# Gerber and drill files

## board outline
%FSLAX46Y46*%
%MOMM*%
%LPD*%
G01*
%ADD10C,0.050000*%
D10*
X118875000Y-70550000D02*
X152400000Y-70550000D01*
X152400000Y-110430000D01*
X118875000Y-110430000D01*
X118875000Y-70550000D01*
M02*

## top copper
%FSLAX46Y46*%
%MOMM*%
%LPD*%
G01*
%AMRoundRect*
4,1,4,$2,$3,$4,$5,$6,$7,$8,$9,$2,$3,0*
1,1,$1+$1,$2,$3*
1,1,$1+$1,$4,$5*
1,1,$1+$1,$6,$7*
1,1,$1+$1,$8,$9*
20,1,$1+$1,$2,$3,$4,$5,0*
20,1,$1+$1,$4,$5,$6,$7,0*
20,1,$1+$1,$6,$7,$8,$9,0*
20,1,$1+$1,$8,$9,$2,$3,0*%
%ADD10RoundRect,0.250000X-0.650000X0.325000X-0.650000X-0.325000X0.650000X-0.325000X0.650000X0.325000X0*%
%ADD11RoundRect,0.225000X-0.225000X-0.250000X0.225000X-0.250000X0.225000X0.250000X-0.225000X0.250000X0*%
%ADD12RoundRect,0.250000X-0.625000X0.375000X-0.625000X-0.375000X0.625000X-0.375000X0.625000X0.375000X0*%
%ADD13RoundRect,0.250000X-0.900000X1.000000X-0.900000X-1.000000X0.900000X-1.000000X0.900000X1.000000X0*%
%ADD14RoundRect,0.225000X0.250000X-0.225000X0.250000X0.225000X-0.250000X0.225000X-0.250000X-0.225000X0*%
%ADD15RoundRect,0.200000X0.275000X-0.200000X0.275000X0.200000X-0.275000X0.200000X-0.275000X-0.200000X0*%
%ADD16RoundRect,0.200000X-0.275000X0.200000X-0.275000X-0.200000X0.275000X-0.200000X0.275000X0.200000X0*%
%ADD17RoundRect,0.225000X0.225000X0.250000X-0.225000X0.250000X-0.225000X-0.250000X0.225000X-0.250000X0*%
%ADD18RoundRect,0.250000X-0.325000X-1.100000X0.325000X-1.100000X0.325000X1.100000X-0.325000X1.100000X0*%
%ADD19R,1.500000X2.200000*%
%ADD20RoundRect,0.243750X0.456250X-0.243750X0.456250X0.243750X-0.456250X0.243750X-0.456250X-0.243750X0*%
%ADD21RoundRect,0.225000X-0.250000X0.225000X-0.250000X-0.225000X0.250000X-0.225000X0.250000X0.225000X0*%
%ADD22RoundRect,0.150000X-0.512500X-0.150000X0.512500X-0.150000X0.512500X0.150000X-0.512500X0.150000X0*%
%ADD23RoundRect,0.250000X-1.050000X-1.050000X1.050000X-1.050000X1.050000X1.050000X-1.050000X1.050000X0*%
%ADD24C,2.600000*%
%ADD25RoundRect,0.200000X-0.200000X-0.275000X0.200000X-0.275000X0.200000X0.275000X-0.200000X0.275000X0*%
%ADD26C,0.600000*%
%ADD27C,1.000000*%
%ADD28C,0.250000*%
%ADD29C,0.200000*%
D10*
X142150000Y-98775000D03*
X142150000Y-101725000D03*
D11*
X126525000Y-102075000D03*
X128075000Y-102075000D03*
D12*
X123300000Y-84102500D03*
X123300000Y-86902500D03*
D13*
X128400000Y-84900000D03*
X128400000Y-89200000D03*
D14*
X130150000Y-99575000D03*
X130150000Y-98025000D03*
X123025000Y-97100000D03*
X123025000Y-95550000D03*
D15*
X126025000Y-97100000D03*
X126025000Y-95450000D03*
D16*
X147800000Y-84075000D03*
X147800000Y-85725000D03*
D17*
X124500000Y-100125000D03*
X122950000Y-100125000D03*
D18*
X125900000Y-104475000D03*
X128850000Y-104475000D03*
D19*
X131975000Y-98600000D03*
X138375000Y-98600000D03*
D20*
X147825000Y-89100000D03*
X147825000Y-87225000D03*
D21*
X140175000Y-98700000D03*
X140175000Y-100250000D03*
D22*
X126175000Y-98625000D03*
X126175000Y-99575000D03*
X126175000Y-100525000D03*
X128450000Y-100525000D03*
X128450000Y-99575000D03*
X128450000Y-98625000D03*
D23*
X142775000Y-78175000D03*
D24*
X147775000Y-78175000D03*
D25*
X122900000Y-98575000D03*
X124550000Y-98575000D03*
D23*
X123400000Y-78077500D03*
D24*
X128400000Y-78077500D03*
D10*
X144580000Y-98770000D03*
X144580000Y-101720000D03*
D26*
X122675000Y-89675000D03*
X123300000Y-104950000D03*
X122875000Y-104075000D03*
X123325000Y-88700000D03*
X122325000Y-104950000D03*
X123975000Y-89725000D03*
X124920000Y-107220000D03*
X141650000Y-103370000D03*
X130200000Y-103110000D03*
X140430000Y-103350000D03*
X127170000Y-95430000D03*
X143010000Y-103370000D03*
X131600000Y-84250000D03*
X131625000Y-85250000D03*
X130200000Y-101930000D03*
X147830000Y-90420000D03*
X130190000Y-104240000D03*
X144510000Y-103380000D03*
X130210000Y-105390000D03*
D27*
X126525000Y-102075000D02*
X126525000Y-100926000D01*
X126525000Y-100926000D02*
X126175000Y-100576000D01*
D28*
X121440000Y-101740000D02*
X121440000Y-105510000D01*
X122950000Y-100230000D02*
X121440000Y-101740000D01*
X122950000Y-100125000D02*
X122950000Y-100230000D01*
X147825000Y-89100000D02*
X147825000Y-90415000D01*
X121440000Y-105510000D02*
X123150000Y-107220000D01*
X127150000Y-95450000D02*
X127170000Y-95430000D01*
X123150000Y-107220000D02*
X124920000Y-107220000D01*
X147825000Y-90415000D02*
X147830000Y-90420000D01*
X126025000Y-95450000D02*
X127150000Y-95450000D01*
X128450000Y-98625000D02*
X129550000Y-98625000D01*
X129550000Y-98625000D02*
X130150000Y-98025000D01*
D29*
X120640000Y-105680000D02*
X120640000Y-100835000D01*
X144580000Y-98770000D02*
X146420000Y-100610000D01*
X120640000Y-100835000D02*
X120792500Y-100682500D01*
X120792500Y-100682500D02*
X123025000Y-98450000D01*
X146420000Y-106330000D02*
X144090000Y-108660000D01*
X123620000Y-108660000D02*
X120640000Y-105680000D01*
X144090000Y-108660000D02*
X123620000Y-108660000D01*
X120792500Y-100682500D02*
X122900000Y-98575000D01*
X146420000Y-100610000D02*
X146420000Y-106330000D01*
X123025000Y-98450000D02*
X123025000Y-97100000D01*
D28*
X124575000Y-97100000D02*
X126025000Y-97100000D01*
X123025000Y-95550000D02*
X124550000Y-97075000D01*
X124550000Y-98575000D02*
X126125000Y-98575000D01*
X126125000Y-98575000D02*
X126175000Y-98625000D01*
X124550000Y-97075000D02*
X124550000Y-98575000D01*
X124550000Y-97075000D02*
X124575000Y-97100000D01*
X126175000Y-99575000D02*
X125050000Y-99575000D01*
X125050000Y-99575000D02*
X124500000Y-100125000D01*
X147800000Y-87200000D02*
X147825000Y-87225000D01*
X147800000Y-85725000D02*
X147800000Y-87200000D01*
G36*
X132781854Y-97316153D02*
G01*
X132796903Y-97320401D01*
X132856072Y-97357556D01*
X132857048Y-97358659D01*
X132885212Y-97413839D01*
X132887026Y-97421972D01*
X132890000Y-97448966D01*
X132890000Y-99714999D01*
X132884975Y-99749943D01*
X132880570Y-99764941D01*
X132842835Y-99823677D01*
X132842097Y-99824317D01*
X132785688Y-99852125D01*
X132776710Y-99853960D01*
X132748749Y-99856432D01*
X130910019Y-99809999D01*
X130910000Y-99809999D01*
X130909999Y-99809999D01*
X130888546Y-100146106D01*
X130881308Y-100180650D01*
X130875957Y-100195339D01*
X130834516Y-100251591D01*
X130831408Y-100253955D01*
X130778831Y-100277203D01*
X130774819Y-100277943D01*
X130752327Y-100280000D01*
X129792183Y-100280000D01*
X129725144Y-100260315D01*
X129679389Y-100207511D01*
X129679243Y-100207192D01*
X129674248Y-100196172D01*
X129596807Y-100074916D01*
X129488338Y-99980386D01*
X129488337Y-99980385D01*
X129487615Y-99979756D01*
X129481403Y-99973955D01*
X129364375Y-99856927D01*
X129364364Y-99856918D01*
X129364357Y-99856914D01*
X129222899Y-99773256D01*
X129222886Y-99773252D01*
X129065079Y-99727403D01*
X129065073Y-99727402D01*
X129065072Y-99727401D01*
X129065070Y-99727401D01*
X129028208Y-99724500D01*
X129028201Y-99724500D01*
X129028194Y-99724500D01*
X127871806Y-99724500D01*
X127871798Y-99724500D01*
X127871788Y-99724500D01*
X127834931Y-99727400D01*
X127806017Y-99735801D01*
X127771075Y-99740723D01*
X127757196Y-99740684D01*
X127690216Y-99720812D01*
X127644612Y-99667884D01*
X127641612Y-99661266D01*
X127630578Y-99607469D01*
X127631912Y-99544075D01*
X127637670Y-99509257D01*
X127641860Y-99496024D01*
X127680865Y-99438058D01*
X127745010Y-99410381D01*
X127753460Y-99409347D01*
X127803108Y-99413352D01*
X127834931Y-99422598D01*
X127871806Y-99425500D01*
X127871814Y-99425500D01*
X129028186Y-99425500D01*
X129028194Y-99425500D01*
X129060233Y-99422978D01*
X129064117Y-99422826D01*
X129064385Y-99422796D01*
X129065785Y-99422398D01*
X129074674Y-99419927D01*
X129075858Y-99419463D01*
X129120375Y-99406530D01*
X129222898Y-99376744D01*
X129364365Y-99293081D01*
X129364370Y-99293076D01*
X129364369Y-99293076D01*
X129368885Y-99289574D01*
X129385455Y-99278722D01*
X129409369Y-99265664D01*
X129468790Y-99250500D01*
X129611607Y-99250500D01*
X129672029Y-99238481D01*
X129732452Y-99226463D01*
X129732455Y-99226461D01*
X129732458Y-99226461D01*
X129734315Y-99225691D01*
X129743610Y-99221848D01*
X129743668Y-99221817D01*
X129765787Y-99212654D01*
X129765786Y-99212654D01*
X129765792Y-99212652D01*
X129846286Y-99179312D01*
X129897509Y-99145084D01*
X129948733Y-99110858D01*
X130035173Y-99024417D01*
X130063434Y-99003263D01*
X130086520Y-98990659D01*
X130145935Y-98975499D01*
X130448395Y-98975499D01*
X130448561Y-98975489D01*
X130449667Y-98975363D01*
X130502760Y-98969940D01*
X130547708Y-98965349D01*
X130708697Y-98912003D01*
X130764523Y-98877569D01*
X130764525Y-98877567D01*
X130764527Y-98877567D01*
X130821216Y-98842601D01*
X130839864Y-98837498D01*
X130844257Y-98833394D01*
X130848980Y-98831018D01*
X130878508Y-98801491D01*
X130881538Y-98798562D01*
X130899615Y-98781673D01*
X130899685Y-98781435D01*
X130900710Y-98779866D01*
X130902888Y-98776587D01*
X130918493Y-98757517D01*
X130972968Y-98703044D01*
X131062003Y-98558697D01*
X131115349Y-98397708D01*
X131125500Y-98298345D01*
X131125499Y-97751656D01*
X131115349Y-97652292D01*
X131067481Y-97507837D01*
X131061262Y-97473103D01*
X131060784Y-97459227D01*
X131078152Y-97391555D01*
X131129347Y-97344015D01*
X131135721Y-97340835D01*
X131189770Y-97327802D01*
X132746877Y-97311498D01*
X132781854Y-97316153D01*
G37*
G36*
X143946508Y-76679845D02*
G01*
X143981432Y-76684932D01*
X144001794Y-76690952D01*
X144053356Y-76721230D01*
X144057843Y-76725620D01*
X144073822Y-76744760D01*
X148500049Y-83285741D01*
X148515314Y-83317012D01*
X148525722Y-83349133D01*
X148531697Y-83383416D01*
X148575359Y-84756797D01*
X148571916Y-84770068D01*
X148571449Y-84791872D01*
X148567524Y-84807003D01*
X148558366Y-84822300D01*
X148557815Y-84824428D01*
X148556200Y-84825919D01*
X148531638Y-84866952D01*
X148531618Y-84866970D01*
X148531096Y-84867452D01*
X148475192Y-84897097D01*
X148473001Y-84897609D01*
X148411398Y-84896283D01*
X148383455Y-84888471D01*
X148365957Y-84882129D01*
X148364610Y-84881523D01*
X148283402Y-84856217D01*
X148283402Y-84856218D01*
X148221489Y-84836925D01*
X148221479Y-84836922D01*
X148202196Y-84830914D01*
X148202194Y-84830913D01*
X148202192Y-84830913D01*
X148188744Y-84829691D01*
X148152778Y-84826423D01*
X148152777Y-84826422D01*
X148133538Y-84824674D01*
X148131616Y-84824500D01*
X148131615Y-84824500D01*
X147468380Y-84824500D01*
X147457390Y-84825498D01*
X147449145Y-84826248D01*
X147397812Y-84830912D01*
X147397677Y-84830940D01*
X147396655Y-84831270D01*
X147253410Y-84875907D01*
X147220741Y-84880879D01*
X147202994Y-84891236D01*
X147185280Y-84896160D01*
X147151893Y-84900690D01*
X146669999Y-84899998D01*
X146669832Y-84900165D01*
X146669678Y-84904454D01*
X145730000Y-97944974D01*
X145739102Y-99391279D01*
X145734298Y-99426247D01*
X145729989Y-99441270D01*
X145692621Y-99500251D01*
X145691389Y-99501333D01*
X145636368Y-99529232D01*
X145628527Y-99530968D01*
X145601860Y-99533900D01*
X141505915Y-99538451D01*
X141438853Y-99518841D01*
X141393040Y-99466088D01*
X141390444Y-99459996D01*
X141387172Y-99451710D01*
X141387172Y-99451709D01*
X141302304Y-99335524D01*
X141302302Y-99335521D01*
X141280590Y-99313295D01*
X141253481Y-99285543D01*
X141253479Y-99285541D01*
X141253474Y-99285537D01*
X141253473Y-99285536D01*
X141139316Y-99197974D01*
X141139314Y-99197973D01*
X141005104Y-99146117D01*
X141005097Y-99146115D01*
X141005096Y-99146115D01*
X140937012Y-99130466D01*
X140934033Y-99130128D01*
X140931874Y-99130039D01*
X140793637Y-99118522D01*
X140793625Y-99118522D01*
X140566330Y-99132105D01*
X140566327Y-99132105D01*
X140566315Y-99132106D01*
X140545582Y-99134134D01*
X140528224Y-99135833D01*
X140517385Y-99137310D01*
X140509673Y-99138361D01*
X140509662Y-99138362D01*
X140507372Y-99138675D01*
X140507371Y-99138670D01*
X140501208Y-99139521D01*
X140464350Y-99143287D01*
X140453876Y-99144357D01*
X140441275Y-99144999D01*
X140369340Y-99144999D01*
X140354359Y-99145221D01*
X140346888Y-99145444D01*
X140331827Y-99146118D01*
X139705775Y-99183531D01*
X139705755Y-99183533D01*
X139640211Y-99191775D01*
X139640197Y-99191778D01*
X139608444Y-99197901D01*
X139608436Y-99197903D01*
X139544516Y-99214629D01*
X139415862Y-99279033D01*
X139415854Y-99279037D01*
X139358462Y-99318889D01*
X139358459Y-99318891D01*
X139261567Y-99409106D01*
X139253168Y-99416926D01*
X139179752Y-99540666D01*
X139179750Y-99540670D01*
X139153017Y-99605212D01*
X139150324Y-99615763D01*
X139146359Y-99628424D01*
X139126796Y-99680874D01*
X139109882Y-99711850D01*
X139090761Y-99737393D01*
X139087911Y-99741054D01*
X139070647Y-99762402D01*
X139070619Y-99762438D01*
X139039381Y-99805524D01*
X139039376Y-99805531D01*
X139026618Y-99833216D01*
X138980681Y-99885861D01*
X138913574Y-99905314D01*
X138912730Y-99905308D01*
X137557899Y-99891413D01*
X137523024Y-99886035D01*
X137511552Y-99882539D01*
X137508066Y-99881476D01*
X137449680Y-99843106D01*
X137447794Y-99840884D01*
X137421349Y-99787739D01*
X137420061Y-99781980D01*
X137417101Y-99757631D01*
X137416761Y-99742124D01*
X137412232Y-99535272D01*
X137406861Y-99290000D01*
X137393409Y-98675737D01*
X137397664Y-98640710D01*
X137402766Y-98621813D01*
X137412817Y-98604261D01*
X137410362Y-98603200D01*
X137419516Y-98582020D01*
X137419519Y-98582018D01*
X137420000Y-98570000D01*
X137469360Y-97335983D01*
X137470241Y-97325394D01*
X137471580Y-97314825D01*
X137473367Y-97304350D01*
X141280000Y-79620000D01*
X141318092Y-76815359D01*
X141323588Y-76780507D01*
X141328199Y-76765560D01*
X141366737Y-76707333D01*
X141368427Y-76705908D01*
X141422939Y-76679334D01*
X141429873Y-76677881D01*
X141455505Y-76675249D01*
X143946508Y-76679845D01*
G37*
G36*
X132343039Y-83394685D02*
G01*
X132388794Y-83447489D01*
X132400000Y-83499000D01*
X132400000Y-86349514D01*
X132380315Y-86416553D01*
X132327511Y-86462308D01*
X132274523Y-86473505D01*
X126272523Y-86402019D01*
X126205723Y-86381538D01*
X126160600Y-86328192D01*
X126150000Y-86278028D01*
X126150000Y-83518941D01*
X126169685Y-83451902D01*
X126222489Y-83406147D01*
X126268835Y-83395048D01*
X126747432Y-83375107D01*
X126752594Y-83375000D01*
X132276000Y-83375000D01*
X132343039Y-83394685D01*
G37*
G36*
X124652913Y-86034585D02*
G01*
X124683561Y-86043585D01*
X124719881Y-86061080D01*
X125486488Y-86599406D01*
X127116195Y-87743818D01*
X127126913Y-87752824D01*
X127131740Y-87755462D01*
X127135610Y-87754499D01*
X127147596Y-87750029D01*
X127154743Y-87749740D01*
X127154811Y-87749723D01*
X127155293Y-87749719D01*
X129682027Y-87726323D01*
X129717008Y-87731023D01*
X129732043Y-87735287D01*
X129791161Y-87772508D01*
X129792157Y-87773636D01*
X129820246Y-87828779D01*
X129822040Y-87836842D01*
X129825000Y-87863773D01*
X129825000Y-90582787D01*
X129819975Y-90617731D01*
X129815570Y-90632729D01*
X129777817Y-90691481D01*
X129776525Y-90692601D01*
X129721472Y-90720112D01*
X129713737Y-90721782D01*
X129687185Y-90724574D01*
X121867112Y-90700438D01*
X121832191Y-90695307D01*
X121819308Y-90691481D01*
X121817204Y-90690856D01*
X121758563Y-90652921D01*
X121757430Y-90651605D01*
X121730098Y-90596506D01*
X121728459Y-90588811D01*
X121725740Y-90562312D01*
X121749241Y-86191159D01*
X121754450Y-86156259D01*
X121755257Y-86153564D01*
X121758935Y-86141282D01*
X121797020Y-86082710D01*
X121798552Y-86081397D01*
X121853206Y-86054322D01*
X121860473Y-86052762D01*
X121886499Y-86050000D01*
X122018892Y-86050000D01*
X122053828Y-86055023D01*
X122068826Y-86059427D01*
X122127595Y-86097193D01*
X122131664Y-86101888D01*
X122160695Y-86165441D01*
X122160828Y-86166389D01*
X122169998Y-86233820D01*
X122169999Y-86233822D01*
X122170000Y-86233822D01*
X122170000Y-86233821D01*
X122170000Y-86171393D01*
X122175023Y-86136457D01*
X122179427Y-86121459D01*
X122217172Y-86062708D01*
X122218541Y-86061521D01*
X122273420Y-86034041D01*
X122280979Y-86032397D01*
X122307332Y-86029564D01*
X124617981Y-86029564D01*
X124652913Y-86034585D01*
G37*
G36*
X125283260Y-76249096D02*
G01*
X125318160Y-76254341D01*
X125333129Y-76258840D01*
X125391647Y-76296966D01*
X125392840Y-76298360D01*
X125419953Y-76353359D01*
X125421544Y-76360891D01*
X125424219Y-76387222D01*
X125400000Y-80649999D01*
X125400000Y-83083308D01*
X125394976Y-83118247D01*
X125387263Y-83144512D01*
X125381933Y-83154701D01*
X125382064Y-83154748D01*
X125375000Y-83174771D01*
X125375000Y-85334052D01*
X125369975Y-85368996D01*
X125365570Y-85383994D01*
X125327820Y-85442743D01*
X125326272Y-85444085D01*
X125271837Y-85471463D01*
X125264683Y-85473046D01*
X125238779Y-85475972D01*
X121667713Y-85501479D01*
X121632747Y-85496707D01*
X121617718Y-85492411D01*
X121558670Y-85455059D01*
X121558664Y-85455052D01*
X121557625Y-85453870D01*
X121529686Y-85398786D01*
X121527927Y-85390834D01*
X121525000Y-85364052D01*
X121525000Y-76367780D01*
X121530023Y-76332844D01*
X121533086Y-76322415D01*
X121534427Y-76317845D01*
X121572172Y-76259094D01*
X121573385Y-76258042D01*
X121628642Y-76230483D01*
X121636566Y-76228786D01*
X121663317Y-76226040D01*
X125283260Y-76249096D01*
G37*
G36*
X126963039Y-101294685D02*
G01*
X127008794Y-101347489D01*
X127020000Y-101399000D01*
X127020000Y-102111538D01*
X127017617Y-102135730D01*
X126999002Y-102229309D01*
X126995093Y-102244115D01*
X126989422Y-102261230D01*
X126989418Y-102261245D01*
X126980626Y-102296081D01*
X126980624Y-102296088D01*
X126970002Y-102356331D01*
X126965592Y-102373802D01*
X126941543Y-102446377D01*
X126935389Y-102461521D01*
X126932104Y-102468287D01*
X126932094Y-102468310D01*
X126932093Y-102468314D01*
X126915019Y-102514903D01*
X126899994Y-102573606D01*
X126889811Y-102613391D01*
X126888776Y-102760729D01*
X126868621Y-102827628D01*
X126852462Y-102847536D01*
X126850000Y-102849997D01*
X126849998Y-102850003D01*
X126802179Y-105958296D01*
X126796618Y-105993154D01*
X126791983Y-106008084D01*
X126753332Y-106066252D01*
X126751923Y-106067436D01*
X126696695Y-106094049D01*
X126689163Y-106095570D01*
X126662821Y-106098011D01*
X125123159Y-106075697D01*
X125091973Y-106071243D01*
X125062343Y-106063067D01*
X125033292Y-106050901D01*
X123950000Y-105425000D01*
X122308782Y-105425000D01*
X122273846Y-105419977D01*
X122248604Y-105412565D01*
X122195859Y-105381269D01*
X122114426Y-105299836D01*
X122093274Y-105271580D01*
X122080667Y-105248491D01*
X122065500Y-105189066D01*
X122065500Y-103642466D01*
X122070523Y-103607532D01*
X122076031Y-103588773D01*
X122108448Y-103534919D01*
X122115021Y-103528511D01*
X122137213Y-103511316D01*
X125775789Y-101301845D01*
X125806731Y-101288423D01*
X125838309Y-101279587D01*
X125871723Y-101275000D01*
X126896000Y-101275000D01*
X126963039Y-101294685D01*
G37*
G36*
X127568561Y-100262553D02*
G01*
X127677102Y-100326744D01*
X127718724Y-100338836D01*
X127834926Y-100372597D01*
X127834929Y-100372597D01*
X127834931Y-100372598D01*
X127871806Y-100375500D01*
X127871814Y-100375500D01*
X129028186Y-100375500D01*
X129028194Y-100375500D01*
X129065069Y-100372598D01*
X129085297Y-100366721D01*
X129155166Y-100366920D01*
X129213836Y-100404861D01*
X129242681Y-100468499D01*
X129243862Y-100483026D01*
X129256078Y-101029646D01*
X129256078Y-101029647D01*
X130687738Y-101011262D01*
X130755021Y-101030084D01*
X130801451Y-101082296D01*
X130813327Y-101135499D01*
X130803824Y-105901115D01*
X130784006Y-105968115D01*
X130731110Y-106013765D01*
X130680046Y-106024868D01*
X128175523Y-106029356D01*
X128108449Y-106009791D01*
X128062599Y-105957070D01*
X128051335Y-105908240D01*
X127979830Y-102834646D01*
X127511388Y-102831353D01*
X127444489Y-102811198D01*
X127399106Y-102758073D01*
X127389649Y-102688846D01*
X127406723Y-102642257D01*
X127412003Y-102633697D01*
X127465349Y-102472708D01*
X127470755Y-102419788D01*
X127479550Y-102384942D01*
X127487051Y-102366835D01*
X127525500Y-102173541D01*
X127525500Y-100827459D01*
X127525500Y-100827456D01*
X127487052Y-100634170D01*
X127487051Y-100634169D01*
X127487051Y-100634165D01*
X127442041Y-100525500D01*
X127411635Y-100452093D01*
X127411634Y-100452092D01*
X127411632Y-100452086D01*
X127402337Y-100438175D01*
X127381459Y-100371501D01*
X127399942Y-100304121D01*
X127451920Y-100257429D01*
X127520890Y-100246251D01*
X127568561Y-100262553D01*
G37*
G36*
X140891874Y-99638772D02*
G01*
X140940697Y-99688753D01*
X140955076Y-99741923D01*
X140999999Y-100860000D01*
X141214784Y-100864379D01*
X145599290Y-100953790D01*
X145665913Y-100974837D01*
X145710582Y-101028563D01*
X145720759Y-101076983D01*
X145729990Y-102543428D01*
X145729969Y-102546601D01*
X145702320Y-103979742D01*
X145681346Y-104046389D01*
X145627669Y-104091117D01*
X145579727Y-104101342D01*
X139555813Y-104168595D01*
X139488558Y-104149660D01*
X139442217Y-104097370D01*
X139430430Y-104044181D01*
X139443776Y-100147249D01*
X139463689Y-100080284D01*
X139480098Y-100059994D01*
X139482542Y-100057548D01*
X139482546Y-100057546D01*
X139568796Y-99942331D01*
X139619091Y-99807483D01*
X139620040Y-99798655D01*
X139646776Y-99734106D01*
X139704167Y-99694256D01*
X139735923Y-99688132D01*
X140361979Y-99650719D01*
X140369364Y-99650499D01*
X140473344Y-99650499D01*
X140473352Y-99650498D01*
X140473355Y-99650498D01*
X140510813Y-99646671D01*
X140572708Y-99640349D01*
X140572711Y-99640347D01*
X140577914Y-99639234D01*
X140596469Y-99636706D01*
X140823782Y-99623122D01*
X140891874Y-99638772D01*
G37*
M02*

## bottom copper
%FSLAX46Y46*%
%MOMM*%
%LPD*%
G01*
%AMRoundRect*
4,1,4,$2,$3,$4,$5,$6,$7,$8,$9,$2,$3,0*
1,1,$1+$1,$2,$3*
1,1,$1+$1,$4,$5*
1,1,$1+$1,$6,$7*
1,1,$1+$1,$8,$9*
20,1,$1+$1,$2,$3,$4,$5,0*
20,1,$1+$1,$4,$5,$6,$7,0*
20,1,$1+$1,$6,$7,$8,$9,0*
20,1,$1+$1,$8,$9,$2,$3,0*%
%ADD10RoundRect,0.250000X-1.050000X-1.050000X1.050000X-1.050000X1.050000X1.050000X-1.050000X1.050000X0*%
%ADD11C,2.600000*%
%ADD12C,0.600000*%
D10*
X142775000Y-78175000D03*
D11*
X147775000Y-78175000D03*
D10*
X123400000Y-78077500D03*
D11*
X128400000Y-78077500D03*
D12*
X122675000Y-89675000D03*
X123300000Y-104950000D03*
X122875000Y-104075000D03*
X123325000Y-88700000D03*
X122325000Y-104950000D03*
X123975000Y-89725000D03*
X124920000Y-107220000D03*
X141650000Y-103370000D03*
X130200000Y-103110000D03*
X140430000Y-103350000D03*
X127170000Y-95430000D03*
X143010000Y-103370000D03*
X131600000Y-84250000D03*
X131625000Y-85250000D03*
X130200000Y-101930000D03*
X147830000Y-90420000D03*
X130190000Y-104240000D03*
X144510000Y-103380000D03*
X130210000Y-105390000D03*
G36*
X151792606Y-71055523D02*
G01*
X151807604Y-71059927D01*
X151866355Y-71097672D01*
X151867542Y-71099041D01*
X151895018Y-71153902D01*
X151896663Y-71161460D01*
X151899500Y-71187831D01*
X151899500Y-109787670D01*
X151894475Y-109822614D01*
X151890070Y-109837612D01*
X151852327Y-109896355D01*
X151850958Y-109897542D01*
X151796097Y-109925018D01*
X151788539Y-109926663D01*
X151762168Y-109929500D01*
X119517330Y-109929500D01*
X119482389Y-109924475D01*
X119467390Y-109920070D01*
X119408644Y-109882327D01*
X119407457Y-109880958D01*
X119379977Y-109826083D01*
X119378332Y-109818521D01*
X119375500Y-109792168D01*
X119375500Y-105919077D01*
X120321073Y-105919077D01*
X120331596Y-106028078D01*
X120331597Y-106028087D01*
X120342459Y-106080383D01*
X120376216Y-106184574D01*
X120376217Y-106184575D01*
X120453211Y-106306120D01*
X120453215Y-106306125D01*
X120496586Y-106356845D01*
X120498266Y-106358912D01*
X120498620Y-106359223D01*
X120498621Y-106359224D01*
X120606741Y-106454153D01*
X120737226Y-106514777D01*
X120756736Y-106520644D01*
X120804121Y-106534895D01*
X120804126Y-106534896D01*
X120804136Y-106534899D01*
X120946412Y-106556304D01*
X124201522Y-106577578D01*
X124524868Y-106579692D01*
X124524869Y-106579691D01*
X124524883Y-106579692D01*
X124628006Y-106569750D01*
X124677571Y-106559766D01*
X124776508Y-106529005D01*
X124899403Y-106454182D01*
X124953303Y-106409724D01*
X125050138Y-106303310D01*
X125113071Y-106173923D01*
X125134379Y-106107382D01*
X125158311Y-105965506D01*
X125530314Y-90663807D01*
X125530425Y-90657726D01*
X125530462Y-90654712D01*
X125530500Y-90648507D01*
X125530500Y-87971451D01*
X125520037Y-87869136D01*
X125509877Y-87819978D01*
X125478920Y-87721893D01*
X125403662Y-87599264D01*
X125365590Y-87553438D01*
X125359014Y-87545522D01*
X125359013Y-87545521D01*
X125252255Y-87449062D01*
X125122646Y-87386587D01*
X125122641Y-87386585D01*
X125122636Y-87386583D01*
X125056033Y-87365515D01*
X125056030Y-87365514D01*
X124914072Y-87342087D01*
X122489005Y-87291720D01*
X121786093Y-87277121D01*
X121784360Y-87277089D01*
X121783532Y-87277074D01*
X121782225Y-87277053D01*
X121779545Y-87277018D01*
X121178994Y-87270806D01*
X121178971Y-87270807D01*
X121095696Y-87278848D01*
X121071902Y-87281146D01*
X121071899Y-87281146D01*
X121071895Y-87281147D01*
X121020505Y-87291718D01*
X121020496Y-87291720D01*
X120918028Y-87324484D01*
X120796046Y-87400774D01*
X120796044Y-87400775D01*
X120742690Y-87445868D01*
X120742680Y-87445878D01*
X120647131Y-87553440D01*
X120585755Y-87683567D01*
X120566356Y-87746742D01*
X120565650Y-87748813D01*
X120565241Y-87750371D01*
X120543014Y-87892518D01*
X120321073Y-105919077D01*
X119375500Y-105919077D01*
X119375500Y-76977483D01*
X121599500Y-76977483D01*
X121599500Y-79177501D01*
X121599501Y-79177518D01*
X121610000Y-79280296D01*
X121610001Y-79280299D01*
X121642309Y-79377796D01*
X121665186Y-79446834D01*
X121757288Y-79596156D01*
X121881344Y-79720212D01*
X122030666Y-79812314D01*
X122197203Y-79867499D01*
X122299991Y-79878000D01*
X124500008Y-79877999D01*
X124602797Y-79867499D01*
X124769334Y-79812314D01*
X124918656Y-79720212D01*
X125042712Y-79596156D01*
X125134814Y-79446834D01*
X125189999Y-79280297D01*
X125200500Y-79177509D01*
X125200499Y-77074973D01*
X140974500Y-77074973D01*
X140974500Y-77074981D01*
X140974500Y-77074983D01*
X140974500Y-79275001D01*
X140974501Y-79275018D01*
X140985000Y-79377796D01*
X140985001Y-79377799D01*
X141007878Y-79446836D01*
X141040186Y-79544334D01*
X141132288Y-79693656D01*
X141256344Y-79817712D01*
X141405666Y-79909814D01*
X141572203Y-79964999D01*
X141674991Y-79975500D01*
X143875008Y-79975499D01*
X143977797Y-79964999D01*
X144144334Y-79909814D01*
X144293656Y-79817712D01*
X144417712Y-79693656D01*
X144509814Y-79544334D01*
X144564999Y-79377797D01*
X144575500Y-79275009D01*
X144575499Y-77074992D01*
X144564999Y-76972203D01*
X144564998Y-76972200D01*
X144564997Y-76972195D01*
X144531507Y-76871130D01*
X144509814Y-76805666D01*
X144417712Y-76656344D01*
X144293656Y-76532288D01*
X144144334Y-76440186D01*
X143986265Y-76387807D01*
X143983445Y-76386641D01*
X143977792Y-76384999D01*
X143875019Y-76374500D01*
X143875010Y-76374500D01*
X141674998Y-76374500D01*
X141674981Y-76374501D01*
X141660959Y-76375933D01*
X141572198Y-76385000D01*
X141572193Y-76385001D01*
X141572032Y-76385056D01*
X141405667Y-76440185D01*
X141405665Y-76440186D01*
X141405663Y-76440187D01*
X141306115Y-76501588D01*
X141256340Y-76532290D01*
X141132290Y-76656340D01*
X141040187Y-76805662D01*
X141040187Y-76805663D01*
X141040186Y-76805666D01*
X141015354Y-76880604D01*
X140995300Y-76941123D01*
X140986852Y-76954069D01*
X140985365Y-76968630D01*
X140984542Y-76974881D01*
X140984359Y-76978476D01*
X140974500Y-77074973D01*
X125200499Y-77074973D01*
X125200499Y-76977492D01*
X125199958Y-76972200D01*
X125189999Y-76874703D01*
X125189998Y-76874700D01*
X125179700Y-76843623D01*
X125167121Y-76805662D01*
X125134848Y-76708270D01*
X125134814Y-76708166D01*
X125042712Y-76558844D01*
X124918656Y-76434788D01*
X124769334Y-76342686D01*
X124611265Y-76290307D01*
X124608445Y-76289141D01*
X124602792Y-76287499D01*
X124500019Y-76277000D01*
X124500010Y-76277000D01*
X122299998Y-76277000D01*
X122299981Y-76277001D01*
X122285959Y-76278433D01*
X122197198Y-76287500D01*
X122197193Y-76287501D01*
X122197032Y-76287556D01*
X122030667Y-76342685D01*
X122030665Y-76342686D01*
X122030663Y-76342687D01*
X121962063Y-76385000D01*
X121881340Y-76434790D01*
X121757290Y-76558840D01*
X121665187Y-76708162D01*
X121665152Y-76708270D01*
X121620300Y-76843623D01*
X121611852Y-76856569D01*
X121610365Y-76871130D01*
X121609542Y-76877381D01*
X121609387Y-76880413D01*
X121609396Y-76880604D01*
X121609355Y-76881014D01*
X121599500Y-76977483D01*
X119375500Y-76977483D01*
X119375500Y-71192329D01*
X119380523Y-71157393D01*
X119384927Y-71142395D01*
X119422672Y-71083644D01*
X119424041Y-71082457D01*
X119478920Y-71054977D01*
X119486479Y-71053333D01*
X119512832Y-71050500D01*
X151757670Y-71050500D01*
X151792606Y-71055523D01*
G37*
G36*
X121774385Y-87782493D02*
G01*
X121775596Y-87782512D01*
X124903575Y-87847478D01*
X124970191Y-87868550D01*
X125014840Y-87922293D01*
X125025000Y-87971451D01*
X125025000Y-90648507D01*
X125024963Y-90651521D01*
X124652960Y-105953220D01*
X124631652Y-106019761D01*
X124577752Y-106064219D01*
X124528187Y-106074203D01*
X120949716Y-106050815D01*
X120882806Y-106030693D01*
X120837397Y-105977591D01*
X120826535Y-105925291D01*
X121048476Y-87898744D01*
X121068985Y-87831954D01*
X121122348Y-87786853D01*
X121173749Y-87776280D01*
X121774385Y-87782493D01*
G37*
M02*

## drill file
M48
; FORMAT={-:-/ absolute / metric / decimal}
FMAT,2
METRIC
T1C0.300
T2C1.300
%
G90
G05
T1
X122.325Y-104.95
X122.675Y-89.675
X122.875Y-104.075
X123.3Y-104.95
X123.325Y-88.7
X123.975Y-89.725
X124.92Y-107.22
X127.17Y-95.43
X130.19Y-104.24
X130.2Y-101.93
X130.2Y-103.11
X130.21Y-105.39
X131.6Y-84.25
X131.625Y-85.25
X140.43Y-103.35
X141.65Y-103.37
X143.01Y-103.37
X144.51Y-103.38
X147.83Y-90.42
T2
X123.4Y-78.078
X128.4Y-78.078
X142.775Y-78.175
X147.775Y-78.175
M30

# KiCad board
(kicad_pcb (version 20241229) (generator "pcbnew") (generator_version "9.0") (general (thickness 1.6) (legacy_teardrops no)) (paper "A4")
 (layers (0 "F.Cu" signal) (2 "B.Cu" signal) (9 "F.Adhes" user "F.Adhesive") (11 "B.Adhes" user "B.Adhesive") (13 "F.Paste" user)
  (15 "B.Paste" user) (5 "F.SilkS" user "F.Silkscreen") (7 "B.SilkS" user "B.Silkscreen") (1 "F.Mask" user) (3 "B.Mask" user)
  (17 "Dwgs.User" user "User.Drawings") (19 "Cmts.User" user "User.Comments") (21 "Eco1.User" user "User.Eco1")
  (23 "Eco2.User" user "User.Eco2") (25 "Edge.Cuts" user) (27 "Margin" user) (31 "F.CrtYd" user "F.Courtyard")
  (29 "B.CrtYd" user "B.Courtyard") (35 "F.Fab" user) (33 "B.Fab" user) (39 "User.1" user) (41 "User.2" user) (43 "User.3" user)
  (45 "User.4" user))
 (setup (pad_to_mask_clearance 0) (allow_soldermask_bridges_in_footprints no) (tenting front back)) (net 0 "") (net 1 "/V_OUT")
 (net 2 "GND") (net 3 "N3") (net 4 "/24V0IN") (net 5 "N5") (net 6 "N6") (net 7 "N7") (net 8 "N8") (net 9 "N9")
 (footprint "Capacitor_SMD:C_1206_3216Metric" (layer "F.Cu") (at 142.15 100.25 -90)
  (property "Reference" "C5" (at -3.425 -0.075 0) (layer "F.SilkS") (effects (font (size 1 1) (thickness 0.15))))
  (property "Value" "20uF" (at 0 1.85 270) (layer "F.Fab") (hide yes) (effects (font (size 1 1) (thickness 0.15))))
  (pad "1" smd roundrect (at -1.475 0 270) (size 1.15 1.8) (layers "F.Cu" "F.Mask" "F.Paste") (roundrect_rratio 0.217391) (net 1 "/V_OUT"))
  (pad "2" smd roundrect (at 1.475 0 270) (size 1.15 1.8) (layers "F.Cu" "F.Mask" "F.Paste") (roundrect_rratio 0.217391) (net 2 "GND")))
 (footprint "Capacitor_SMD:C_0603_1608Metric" (layer "F.Cu") (at 127.3 102.075)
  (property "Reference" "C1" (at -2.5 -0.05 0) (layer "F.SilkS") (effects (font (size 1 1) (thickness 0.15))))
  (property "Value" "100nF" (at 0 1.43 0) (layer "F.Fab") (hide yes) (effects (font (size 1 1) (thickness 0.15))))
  (pad "1" smd roundrect (at -0.775 0) (size 0.9 0.95) (layers "F.Cu" "F.Mask" "F.Paste") (roundrect_rratio 0.25) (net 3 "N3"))
  (pad "2" smd roundrect (at 0.775 0) (size 0.9 0.95) (layers "F.Cu" "F.Mask" "F.Paste") (roundrect_rratio 0.25) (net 2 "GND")))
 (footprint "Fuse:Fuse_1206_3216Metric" (layer "F.Cu") (at 123.3 85.5025 -90)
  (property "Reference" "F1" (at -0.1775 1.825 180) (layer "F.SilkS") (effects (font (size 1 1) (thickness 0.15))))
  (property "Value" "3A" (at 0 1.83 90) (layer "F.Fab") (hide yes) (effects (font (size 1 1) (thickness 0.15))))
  (pad "1" smd roundrect (at -1.4 0 270) (size 1.25 1.75) (layers "F.Cu" "F.Mask" "F.Paste") (roundrect_rratio 0.2) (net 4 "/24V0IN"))
  (pad "2" smd roundrect (at 1.4 0 270) (size 1.25 1.75) (layers "F.Cu" "F.Mask" "F.Paste") (roundrect_rratio 0.2) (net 3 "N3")))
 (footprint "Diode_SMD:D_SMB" (layer "F.Cu") (at 128.4 87.05 -90)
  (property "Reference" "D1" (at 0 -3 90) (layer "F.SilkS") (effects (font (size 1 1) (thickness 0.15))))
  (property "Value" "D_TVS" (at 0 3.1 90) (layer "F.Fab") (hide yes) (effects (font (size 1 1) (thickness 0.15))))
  (pad "1" smd roundrect (at -2.15 0 270) (size 2.5 2.3) (layers "F.Cu" "F.Mask" "F.Paste") (roundrect_rratio 0.1086956522) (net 2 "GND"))
  (pad "2" smd roundrect (at 2.15 0 270) (size 2.5 2.3) (layers "F.Cu" "F.Mask" "F.Paste") (roundrect_rratio 0.1086956522) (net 3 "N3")))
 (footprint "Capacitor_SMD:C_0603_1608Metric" (layer "F.Cu") (at 130.15 98.8 90)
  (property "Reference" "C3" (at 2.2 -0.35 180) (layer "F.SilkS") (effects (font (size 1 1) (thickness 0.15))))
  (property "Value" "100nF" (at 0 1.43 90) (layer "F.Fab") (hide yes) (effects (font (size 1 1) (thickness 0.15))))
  (pad "1" smd roundrect (at -0.775 0 90) (size 0.9 0.95) (layers "F.Cu" "F.Mask" "F.Paste") (roundrect_rratio 0.25) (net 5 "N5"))
  (pad "2" smd roundrect (at 0.775 0 90) (size 0.9 0.95) (layers "F.Cu" "F.Mask" "F.Paste") (roundrect_rratio 0.25) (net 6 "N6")))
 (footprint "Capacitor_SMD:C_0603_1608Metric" (layer "F.Cu") (at 123.025 96.325 90)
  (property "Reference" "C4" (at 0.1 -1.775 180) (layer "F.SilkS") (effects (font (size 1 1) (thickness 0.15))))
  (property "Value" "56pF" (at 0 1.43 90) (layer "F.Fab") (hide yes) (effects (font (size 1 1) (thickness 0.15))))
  (pad "1" smd roundrect (at -0.775 0 90) (size 0.9 0.95) (layers "F.Cu" "F.Mask" "F.Paste") (roundrect_rratio 0.25) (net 1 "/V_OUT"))
  (pad "2" smd roundrect (at 0.775 0 90) (size 0.9 0.95) (layers "F.Cu" "F.Mask" "F.Paste") (roundrect_rratio 0.25) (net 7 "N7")))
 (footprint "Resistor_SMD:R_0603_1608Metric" (layer "F.Cu") (at 126.025 96.275 90)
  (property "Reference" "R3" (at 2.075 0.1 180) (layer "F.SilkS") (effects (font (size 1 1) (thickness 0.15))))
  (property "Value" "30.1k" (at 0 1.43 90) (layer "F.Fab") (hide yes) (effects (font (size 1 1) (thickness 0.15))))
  (pad "1" smd roundrect (at -0.825 0 90) (size 0.8 0.95) (layers "F.Cu" "F.Mask" "F.Paste") (roundrect_rratio 0.25) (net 7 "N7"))
  (pad "2" smd roundrect (at 0.825 0 90) (size 0.8 0.95) (layers "F.Cu" "F.Mask" "F.Paste") (roundrect_rratio 0.25) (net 2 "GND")))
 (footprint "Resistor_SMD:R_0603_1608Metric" (layer "F.Cu") (at 147.8 84.9 -90)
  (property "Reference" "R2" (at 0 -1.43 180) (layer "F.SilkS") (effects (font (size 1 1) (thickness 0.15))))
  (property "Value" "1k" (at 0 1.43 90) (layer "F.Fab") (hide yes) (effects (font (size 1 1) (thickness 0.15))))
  (pad "1" smd roundrect (at -0.825 0 270) (size 0.8 0.95) (layers "F.Cu" "F.Mask" "F.Paste") (roundrect_rratio 0.25) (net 1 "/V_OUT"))
  (pad "2" smd roundrect (at 0.825 0 270) (size 0.8 0.95) (layers "F.Cu" "F.Mask" "F.Paste") (roundrect_rratio 0.25) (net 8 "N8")))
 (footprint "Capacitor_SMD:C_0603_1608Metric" (layer "F.Cu") (at 123.725 100.125 180)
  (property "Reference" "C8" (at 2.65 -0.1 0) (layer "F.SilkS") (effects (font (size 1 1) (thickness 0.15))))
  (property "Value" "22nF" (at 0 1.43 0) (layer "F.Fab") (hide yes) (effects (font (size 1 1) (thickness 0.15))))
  (pad "1" smd roundrect (at -0.775 0 180) (size 0.9 0.95) (layers "F.Cu" "F.Mask" "F.Paste") (roundrect_rratio 0.25) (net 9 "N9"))
  (pad "2" smd roundrect (at 0.775 0 180) (size 0.9 0.95) (layers "F.Cu" "F.Mask" "F.Paste") (roundrect_rratio 0.25) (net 2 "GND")))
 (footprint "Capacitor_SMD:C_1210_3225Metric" (layer "F.Cu") (at 127.375 104.475)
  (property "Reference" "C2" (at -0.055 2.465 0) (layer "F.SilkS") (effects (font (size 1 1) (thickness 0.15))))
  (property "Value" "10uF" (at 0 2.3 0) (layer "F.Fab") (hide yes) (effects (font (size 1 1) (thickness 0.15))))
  (pad "1" smd roundrect (at -1.475 0) (size 1.15 2.7) (layers "F.Cu" "F.Mask" "F.Paste") (roundrect_rratio 0.217391) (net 3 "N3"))
  (pad "2" smd roundrect (at 1.475 0) (size 1.15 2.7) (layers "F.Cu" "F.Mask" "F.Paste") (roundrect_rratio 0.217391) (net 2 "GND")))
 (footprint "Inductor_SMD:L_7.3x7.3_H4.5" (layer "F.Cu") (at 135.175 98.6)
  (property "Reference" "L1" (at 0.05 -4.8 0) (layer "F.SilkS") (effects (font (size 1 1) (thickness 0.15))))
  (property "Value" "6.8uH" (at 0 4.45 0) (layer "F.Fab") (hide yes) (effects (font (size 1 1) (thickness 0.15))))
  (pad "1" smd rect (at -3.2 0) (size 1.5 2.2) (layers "F.Cu" "F.Mask" "F.Paste") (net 5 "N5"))
  (pad "2" smd rect (at 3.2 0) (size 1.5 2.2) (layers "F.Cu" "F.Mask" "F.Paste") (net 1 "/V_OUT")))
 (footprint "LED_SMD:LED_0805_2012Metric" (layer "F.Cu") (at 147.825 88.1625 90)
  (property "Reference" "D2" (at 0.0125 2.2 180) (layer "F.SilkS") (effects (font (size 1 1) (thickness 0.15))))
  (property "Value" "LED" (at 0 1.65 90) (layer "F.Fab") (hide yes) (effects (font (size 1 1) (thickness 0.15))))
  (pad "1" smd roundrect (at -0.9375 0 90) (size 0.975 1.4) (layers "F.Cu" "F.Mask" "F.Paste") (roundrect_rratio 0.25) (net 2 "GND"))
  (pad "2" smd roundrect (at 0.9375 0 90) (size 0.975 1.4) (layers "F.Cu" "F.Mask" "F.Paste") (roundrect_rratio 0.25) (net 8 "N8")))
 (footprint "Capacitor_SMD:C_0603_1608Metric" (layer "F.Cu") (at 140.175 99.475 -90)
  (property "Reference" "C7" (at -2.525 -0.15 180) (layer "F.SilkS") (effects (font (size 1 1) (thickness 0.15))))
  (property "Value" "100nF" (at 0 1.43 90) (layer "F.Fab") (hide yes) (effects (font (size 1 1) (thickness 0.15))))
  (pad "1" smd roundrect (at -0.775 0 270) (size 0.9 0.95) (layers "F.Cu" "F.Mask" "F.Paste") (roundrect_rratio 0.25) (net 1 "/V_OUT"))
  (pad "2" smd roundrect (at 0.775 0 270) (size 0.9 0.95) (layers "F.Cu" "F.Mask" "F.Paste") (roundrect_rratio 0.25) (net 2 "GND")))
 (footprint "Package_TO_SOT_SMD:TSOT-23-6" (layer "F.Cu") (at 127.3125 99.575)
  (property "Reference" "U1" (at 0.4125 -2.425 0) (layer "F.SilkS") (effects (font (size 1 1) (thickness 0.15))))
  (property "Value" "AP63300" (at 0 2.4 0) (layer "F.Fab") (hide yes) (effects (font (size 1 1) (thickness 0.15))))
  (pad "1" smd roundrect (at -1.1375 -0.95) (size 1.325 0.6) (layers "F.Cu" "F.Mask" "F.Paste") (roundrect_rratio 0.25) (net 7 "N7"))
  (pad "2" smd roundrect (at -1.1375 0) (size 1.325 0.6) (layers "F.Cu" "F.Mask" "F.Paste") (roundrect_rratio 0.25) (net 9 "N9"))
  (pad "3" smd roundrect (at -1.1375 0.95) (size 1.325 0.6) (layers "F.Cu" "F.Mask" "F.Paste") (roundrect_rratio 0.25) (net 3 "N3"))
  (pad "4" smd roundrect (at 1.1375 0.95) (size 1.325 0.6) (layers "F.Cu" "F.Mask" "F.Paste") (roundrect_rratio 0.25) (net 2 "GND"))
  (pad "5" smd roundrect (at 1.1375 0) (size 1.325 0.6) (layers "F.Cu" "F.Mask" "F.Paste") (roundrect_rratio 0.25) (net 5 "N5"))
  (pad "6" smd roundrect (at 1.1375 -0.95) (size 1.325 0.6) (layers "F.Cu" "F.Mask" "F.Paste") (roundrect_rratio 0.25) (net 6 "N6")))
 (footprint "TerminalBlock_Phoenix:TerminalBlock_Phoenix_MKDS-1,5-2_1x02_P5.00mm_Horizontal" (layer "F.Cu") (at 142.775 78.175)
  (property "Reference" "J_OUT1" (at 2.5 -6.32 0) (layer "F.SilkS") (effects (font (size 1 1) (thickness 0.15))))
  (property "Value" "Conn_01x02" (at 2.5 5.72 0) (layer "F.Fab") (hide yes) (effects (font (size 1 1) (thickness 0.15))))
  (pad "1" thru_hole roundrect (at 0 0) (size 2.6 2.6) (drill 1.3) (layers "*.Cu" "*.Mask") (remove_unused_layers no)
   (roundrect_rratio 0.096154) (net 1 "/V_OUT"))
  (pad "2" thru_hole circle (at 5 0) (size 2.6 2.6) (drill 1.3) (layers "*.Cu" "*.Mask") (remove_unused_layers no) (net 2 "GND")))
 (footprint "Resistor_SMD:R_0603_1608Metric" (layer "F.Cu") (at 123.725 98.575)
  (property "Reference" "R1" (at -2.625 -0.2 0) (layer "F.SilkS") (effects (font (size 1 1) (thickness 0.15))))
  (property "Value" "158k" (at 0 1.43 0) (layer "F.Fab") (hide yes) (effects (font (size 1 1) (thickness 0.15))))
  (pad "1" smd roundrect (at -0.825 0) (size 0.8 0.95) (layers "F.Cu" "F.Mask" "F.Paste") (roundrect_rratio 0.25) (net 1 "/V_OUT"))
  (pad "2" smd roundrect (at 0.825 0) (size 0.8 0.95) (layers "F.Cu" "F.Mask" "F.Paste") (roundrect_rratio 0.25) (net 7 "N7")))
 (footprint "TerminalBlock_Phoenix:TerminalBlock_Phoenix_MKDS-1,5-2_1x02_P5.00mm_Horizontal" (layer "F.Cu") (at 123.4 78.0775)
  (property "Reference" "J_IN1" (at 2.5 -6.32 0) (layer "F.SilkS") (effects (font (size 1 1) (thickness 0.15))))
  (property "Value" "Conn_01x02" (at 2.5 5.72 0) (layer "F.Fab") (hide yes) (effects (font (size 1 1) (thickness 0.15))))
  (pad "1" thru_hole roundrect (at 0 0) (size 2.6 2.6) (drill 1.3) (layers "*.Cu" "*.Mask") (remove_unused_layers no)
   (roundrect_rratio 0.096154) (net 4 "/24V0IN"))
  (pad "2" thru_hole circle (at 5 0) (size 2.6 2.6) (drill 1.3) (layers "*.Cu" "*.Mask") (remove_unused_layers no) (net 2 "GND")))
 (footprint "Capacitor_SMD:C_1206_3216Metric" (layer "F.Cu") (at 144.58 100.245 -90)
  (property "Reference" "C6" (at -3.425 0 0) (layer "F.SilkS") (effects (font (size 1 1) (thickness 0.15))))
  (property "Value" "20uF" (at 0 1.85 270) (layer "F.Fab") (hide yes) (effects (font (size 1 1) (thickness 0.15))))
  (pad "1" smd roundrect (at -1.475 0 270) (size 1.15 1.8) (layers "F.Cu" "F.Mask" "F.Paste") (roundrect_rratio 0.217391) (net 1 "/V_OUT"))
  (pad "2" smd roundrect (at 1.475 0 270) (size 1.15 1.8) (layers "F.Cu" "F.Mask" "F.Paste") (roundrect_rratio 0.217391) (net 2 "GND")))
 (gr_rect (start 118.875 70.55) (end 152.4 110.43) (stroke (width 0.05) (type default)) (fill no) (layer "Edge.Cuts"))
 (segment (start 126.525 102.075) (end 126.525 100.926) (width 1) (layer "F.Cu") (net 3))
 (segment (start 126.525 100.926) (end 126.175 100.576) (width 1) (layer "F.Cu") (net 3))
 (via (at 122.675 89.675) (size 0.6) (drill 0.3) (layers "F.Cu" "B.Cu") (free yes) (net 3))
 (via (at 123.3 104.95) (size 0.6) (drill 0.3) (layers "F.Cu" "B.Cu") (free yes) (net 3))
 (via (at 122.875 104.075) (size 0.6) (drill 0.3) (layers "F.Cu" "B.Cu") (free yes) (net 3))
 (via (at 123.325 88.7) (size 0.6) (drill 0.3) (layers "F.Cu" "B.Cu") (free yes) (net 3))
 (via (at 122.325 104.95) (size 0.6) (drill 0.3) (layers "F.Cu" "B.Cu") (free yes) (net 3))
 (via (at 123.975 89.725) (size 0.6) (drill 0.3) (layers "F.Cu" "B.Cu") (free yes) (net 3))
 (segment (start 121.44 101.74) (end 121.44 105.51) (width 0.25) (layer "F.Cu") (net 2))
 (segment (start 122.95 100.23) (end 121.44 101.74) (width 0.25) (layer "F.Cu") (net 2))
 (segment (start 122.95 100.125) (end 122.95 100.23) (width 0.25) (layer "F.Cu") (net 2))
 (segment (start 147.825 89.1) (end 147.825 90.415) (width 0.25) (layer "F.Cu") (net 2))
 (segment (start 121.44 105.51) (end 123.15 107.22) (width 0.25) (layer "F.Cu") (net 2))
 (segment (start 127.15 95.45) (end 127.17 95.43) (width 0.25) (layer "F.Cu") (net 2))
 (segment (start 123.15 107.22) (end 124.92 107.22) (width 0.25) (layer "F.Cu") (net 2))
 (segment (start 147.825 90.415) (end 147.83 90.42) (width 0.25) (layer "F.Cu") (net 2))
 (segment (start 126.025 95.45) (end 127.15 95.45) (width 0.25) (layer "F.Cu") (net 2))
 (via (at 124.92 107.22) (size 0.6) (drill 0.3) (layers "F.Cu" "B.Cu") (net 2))
 (via (at 141.65 103.37) (size 0.6) (drill 0.3) (layers "F.Cu" "B.Cu") (free yes) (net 2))
 (via (at 130.2 103.11) (size 0.6) (drill 0.3) (layers "F.Cu" "B.Cu") (free yes) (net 2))
 (via (at 140.43 103.35) (size 0.6) (drill 0.3) (layers "F.Cu" "B.Cu") (free yes) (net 2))
 (via (at 127.17 95.43) (size 0.6) (drill 0.3) (layers "F.Cu" "B.Cu") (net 2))
 (via (at 143.01 103.37) (size 0.6) (drill 0.3) (layers "F.Cu" "B.Cu") (free yes) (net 2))
 (via (at 131.6 84.25) (size 0.6) (drill 0.3) (layers "F.Cu" "B.Cu") (free yes) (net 2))
 (via (at 131.625 85.25) (size 0.6) (drill 0.3) (layers "F.Cu" "B.Cu") (free yes) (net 2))
 (via (at 130.2 101.93) (size 0.6) (drill 0.3) (layers "F.Cu" "B.Cu") (free yes) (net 2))
 (via (at 147.83 90.42) (size 0.6) (drill 0.3) (layers "F.Cu" "B.Cu") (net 2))
 (via (at 130.19 104.24) (size 0.6) (drill 0.3) (layers "F.Cu" "B.Cu") (free yes) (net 2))
 (via (at 144.51 103.38) (size 0.6) (drill 0.3) (layers "F.Cu" "B.Cu") (free yes) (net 2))
 (via (at 130.21 105.39) (size 0.6) (drill 0.3) (layers "F.Cu" "B.Cu") (free yes) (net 2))
 (segment (start 128.45 98.625) (end 129.55 98.625) (width 0.25) (layer "F.Cu") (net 6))
 (segment (start 129.55 98.625) (end 130.15 98.025) (width 0.25) (layer "F.Cu") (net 6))
 (segment (start 120.64 105.68) (end 120.64 100.835) (width 0.2) (layer "F.Cu") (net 1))
 (segment (start 144.58 98.77) (end 146.42 100.61) (width 0.2) (layer "F.Cu") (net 1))
 (segment (start 120.64 100.835) (end 120.7925 100.6825) (width 0.2) (layer "F.Cu") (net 1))
 (segment (start 120.7925 100.6825) (end 123.025 98.45) (width 0.2) (layer "F.Cu") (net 1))
 (segment (start 146.42 106.33) (end 144.09 108.66) (width 0.2) (layer "F.Cu") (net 1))
 (segment (start 123.62 108.66) (end 120.64 105.68) (width 0.2) (layer "F.Cu") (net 1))
 (segment (start 144.09 108.66) (end 123.62 108.66) (width 0.2) (layer "F.Cu") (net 1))
 (segment (start 120.7925 100.6825) (end 122.9 98.575) (width 0.2) (layer "F.Cu") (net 1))
 (segment (start 146.42 100.61) (end 146.42 106.33) (width 0.2) (layer "F.Cu") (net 1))
 (segment (start 123.025 98.45) (end 123.025 97.1) (width 0.2) (layer "F.Cu") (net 1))
 (segment (start 124.575 97.1) (end 126.025 97.1) (width 0.25) (layer "F.Cu") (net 7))
 (segment (start 123.025 95.55) (end 124.55 97.075) (width 0.25) (layer "F.Cu") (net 7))
 (segment (start 124.55 98.575) (end 126.125 98.575) (width 0.25) (layer "F.Cu") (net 7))
 (segment (start 126.125 98.575) (end 126.175 98.625) (width 0.25) (layer "F.Cu") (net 7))
 (segment (start 124.55 97.075) (end 124.55 98.575) (width 0.25) (layer "F.Cu") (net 7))
 (segment (start 124.55 97.075) (end 124.575 97.1) (width 0.25) (layer "F.Cu") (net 7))
 (segment (start 126.175 99.575) (end 125.05 99.575) (width 0.25) (layer "F.Cu") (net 9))
 (segment (start 125.05 99.575) (end 124.5 100.125) (width 0.25) (layer "F.Cu") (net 9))
 (segment (start 147.8 87.2) (end 147.825 87.225) (width 0.25) (layer "F.Cu") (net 8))
 (segment (start 147.8 85.725) (end 147.8 87.2) (width 0.25) (layer "F.Cu") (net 8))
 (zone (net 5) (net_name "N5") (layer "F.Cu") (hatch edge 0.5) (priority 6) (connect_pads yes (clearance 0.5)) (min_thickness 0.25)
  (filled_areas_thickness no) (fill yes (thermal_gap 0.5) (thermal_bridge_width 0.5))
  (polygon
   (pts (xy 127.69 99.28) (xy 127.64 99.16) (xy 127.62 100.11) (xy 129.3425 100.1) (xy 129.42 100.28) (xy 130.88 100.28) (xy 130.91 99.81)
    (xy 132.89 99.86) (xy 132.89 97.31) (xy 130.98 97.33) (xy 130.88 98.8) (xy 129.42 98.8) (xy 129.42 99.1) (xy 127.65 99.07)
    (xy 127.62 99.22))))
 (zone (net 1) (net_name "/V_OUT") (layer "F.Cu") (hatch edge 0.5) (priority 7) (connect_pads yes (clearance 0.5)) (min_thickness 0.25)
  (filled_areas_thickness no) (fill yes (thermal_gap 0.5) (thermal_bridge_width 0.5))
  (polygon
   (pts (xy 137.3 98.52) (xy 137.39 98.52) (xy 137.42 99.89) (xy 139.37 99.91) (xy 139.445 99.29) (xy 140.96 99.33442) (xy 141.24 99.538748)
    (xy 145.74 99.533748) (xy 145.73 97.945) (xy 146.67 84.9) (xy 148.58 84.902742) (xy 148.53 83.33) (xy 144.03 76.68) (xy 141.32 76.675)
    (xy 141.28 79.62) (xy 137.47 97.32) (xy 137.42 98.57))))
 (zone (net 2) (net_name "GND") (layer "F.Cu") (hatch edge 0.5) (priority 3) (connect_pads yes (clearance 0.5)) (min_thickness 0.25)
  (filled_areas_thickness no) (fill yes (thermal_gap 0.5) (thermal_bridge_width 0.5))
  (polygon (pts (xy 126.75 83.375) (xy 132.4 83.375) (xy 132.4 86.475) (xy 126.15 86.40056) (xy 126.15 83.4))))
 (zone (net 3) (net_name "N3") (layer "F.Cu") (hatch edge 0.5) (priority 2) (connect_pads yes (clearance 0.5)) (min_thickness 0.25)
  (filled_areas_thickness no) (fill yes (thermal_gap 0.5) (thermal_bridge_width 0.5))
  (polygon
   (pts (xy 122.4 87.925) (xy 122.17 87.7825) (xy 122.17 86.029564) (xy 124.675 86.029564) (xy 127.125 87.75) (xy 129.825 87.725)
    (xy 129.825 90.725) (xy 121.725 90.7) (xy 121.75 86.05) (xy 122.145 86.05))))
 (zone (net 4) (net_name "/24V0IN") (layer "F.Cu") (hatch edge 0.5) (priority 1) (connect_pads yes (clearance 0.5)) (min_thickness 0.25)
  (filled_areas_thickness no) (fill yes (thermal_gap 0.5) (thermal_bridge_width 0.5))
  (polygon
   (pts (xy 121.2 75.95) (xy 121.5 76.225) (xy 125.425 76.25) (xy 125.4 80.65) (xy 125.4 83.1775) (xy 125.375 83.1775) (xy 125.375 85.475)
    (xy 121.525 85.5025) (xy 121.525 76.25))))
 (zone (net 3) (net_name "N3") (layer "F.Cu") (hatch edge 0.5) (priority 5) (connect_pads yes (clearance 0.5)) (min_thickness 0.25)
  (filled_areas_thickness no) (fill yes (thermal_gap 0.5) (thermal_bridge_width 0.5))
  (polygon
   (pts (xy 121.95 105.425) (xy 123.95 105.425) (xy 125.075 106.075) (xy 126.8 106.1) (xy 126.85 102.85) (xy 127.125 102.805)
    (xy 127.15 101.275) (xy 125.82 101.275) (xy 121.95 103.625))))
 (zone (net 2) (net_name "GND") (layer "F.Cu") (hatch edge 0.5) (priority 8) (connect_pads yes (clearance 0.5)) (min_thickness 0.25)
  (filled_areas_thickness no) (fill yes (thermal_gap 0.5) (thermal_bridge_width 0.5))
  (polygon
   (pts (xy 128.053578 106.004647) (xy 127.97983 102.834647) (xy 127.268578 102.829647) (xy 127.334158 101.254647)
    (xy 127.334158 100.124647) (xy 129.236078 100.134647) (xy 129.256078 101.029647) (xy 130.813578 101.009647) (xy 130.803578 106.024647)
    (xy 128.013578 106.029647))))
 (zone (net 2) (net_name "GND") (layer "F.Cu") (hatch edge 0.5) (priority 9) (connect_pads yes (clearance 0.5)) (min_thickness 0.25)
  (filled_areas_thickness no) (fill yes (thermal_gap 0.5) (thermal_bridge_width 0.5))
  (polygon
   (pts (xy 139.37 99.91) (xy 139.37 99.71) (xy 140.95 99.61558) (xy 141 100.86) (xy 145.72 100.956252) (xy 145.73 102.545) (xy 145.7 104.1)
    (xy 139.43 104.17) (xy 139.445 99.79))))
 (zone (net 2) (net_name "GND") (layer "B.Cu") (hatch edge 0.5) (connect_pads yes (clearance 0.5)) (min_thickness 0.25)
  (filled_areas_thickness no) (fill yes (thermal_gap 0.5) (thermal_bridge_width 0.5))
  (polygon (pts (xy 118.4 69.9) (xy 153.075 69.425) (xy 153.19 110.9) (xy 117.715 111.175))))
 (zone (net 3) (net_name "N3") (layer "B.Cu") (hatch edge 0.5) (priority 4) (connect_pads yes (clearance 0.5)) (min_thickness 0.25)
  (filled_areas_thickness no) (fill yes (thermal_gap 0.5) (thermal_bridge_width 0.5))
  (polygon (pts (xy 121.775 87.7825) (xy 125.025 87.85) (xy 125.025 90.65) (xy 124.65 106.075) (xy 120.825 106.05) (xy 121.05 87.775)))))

